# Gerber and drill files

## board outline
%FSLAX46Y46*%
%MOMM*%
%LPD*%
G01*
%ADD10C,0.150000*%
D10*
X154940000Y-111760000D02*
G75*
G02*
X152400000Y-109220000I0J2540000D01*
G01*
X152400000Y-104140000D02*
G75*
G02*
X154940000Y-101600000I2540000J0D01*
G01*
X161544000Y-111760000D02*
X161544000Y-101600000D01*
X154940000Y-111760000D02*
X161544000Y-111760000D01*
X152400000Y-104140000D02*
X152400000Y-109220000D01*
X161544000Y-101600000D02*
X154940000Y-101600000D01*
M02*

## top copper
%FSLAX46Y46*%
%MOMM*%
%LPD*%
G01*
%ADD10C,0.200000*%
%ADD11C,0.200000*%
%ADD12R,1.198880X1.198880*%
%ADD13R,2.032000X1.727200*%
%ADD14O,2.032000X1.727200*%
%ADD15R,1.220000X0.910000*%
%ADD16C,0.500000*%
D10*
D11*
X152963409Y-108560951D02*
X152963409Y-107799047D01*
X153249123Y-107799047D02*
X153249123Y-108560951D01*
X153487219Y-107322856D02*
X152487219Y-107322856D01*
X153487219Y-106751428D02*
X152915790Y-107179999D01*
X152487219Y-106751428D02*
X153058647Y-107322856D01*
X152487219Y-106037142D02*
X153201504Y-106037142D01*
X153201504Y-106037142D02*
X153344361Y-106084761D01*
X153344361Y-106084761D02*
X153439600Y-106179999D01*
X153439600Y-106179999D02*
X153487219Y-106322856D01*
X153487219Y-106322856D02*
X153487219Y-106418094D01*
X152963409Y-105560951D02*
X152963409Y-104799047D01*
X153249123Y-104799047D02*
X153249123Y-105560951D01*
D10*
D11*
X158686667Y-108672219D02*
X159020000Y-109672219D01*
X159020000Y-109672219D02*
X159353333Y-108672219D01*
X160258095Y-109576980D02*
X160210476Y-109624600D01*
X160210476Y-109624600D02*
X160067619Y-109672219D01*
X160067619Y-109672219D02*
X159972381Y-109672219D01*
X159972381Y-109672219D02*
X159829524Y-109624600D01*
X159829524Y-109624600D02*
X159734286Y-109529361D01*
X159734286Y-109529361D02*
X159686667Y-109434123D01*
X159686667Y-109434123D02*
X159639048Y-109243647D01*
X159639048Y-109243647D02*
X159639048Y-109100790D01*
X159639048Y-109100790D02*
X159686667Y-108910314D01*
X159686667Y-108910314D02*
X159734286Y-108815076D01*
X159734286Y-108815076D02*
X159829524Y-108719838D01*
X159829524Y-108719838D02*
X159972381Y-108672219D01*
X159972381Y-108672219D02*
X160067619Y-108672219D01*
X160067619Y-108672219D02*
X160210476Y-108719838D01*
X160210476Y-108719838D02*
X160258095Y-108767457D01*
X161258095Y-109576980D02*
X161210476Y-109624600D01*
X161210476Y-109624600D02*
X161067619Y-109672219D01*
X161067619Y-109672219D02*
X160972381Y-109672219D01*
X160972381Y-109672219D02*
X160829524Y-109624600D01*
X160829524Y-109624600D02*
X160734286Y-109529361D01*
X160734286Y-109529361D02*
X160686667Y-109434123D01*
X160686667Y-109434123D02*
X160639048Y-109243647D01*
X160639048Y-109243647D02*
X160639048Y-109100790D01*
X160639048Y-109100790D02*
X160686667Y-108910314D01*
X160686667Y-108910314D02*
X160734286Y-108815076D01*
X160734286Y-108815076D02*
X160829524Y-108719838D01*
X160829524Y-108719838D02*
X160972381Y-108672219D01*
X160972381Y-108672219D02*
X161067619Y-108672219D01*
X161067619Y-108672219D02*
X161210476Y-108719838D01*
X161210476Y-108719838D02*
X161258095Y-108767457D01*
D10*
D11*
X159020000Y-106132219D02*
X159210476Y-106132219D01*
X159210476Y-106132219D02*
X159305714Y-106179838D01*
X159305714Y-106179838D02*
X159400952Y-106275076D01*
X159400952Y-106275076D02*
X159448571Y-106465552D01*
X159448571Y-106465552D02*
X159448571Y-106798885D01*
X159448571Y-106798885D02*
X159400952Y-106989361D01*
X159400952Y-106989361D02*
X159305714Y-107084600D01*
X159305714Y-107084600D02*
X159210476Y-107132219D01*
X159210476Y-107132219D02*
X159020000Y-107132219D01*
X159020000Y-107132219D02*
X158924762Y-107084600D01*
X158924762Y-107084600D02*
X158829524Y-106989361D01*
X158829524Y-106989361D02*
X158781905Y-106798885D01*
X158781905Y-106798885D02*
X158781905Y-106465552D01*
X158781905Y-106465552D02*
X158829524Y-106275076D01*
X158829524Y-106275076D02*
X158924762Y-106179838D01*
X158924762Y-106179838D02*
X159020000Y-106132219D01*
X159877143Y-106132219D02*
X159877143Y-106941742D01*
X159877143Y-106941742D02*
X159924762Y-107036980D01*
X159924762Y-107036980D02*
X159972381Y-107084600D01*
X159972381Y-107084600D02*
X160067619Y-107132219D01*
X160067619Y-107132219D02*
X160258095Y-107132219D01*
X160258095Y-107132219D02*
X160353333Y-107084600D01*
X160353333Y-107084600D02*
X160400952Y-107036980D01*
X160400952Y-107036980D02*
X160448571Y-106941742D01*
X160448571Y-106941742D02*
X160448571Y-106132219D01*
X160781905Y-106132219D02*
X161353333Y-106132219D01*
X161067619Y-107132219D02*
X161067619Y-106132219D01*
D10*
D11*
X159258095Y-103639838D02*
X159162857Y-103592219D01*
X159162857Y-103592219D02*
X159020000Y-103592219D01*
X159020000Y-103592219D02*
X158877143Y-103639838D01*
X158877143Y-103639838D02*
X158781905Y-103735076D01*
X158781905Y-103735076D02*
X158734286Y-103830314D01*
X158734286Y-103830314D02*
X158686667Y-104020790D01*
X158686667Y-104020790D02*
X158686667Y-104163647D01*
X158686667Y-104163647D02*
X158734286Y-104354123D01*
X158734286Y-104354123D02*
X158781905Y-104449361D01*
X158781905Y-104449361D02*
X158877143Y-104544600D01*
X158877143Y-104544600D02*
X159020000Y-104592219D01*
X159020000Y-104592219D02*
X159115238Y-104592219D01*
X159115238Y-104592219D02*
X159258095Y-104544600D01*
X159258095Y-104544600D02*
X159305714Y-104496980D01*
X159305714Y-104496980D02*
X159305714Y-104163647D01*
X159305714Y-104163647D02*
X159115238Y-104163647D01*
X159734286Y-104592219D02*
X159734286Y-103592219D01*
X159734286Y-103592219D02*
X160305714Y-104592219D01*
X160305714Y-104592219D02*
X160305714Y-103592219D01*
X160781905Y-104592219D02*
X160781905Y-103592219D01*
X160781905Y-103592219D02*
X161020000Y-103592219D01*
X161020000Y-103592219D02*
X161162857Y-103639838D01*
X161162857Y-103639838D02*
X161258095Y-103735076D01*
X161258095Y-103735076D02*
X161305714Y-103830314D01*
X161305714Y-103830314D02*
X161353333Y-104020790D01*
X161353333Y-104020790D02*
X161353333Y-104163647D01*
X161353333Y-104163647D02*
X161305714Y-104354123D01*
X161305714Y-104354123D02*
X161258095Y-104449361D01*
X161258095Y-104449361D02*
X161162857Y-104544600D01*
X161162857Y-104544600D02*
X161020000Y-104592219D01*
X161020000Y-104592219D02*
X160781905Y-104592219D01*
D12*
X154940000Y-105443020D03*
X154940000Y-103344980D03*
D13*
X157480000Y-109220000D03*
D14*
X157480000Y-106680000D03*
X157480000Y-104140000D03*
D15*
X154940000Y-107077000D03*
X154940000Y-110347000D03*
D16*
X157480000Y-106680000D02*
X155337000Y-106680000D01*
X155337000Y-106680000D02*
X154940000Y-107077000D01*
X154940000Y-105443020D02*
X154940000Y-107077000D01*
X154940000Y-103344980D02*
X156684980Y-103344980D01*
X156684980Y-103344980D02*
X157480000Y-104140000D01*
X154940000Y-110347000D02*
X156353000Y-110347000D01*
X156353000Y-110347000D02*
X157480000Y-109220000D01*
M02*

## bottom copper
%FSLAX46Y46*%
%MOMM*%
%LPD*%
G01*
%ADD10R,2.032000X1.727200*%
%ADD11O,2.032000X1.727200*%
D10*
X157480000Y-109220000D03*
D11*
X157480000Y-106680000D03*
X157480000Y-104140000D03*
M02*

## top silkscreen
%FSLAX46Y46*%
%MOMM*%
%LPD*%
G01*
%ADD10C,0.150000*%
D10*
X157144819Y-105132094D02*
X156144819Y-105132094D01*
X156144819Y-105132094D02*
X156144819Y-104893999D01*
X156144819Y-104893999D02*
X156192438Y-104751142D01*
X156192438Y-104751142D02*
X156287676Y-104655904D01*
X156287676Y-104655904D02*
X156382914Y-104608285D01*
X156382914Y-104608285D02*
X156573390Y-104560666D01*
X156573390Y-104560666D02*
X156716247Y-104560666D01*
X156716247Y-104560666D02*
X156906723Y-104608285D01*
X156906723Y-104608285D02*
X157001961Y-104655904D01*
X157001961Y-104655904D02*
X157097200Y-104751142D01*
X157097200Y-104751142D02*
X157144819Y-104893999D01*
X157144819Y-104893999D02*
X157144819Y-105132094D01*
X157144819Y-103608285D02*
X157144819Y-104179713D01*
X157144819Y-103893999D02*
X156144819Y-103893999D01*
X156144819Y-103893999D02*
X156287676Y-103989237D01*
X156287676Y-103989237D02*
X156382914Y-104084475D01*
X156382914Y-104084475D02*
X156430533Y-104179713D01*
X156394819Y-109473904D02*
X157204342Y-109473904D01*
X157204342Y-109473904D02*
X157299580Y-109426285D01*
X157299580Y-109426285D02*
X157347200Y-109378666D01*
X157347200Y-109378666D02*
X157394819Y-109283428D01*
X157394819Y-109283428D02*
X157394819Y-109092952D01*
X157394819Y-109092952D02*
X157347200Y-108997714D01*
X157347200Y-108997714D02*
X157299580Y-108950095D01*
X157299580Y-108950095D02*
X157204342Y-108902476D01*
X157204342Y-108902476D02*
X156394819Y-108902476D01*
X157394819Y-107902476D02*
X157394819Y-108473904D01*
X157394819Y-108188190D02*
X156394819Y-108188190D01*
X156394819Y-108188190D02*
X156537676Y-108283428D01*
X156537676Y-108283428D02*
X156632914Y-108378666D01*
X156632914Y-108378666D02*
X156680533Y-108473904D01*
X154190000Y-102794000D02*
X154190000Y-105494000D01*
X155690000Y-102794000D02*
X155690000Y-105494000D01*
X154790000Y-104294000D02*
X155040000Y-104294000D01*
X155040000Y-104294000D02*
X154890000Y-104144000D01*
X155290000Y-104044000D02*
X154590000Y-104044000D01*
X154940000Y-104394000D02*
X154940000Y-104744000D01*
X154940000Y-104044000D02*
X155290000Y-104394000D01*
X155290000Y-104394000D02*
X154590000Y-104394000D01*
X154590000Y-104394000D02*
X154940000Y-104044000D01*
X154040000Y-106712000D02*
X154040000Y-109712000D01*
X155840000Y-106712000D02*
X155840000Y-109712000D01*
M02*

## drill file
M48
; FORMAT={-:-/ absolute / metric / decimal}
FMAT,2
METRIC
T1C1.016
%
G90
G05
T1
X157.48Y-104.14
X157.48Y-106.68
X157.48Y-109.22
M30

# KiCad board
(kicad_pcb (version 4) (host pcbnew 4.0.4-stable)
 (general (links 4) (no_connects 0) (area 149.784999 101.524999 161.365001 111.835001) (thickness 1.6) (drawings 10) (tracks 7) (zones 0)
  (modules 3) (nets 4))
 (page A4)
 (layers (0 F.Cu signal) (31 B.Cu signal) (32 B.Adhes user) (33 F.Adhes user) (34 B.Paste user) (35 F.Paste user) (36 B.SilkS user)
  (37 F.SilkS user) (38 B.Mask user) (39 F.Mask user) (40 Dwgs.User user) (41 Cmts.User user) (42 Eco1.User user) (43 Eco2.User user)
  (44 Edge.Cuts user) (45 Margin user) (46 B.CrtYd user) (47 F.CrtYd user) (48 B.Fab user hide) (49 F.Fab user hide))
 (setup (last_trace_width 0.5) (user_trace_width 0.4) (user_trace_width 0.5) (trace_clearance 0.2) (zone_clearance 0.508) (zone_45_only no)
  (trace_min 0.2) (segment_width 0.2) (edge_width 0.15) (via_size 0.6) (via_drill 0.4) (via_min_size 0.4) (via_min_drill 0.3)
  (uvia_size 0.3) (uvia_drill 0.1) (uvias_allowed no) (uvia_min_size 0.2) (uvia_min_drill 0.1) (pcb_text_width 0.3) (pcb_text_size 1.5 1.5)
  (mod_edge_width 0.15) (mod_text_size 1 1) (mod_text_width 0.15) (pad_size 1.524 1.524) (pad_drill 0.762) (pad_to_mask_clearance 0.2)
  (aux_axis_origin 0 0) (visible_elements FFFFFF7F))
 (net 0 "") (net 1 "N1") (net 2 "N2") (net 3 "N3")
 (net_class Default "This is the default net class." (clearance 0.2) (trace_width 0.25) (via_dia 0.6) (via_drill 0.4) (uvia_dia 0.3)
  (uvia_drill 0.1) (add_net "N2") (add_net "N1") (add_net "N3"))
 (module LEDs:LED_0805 (layer F.Cu) (at 154.94 104.394 270)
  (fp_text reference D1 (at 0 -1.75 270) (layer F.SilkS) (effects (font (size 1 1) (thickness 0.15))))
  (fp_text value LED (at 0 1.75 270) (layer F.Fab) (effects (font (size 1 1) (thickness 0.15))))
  (fp_line (start -1.6 0.75) (end 1.1 0.75) (layer F.SilkS) (width 0.15))
  (fp_line (start -1.6 -0.75) (end 1.1 -0.75) (layer F.SilkS) (width 0.15))
  (fp_line (start -0.1 0.15) (end -0.1 -0.1) (layer F.SilkS) (width 0.15))
  (fp_line (start -0.1 -0.1) (end -0.25 0.05) (layer F.SilkS) (width 0.15))
  (fp_line (start -0.35 -0.35) (end -0.35 0.35) (layer F.SilkS) (width 0.15))
  (fp_line (start 0 0) (end 0.35 0) (layer F.SilkS) (width 0.15))
  (fp_line (start -0.35 0) (end 0 -0.35) (layer F.SilkS) (width 0.15))
  (fp_line (start 0 -0.35) (end 0 0.35) (layer F.SilkS) (width 0.15))
  (fp_line (start 0 0.35) (end -0.35 0) (layer F.SilkS) (width 0.15))
  (pad 2 smd rect (at 1.04902 0 90) (size 1.19888 1.19888) (layers F.Cu F.Paste F.Mask) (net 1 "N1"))
  (pad 1 smd rect (at -1.04902 0 90) (size 1.19888 1.19888) (layers F.Cu F.Paste F.Mask) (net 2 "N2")))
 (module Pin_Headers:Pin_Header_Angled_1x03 (layer B.Cu) (at 157.48 109.22)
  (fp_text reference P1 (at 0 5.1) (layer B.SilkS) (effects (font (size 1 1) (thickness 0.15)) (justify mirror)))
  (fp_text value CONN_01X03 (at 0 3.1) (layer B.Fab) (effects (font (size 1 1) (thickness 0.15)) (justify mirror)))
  (pad 1 thru_hole rect (at 0 0) (size 2.032 1.7272) (drill 1.016) (layers *.Cu *.Mask) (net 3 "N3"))
  (pad 2 thru_hole oval (at 0 -2.54) (size 2.032 1.7272) (drill 1.016) (layers *.Cu *.Mask) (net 1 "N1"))
  (pad 3 thru_hole oval (at 0 -5.08) (size 2.032 1.7272) (drill 1.016) (layers *.Cu *.Mask) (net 2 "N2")))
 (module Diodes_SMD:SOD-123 (layer F.Cu) (at 154.94 108.712 270)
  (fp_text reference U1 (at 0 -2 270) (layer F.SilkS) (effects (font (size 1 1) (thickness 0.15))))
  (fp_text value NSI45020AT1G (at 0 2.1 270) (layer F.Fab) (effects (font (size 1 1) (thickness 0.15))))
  (fp_line (start -2 0.9) (end 1 0.9) (layer F.SilkS) (width 0.15))
  (fp_line (start -2 -0.9) (end 1 -0.9) (layer F.SilkS) (width 0.15))
  (pad 1 smd rect (at -1.635 0 270) (size 0.91 1.22) (layers F.Cu F.Paste F.Mask) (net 1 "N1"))
  (pad 2 smd rect (at 1.635 0 270) (size 0.91 1.22) (layers F.Cu F.Paste F.Mask) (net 3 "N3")))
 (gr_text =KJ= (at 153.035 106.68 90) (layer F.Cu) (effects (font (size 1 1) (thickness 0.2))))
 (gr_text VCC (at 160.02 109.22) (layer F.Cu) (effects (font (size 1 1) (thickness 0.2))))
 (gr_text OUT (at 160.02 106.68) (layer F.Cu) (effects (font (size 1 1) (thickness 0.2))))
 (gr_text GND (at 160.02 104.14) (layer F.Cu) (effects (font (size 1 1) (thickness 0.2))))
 (gr_arc (start 154.94 109.22) (end 154.94 111.76) (angle 90) (layer Edge.Cuts) (width 0.15))
 (gr_arc (start 154.94 104.14) (end 152.4 104.14) (angle 90) (layer Edge.Cuts) (width 0.15))
 (gr_line (start 161.544 111.76) (end 161.544 101.6) (layer Edge.Cuts) (width 0.15))
 (gr_line (start 154.94 111.76) (end 161.544 111.76) (layer Edge.Cuts) (width 0.15))
 (gr_line (start 152.4 104.14) (end 152.4 109.22) (layer Edge.Cuts) (width 0.15))
 (gr_line (start 161.544 101.6) (end 154.94 101.6) (layer Edge.Cuts) (width 0.15))
 (segment (start 157.48 106.68) (end 155.337 106.68) (width 0.5) (layer F.Cu) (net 1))
 (segment (start 155.337 106.68) (end 154.94 107.077) (width 0.5) (layer F.Cu) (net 1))
 (segment (start 154.94 105.44302) (end 154.94 107.077) (width 0.5) (layer F.Cu) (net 1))
 (segment (start 154.94 103.34498) (end 156.68498 103.34498) (width 0.5) (layer F.Cu) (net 2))
 (segment (start 156.68498 103.34498) (end 157.48 104.14) (width 0.5) (layer F.Cu) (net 2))
 (segment (start 154.94 110.347) (end 156.353 110.347) (width 0.5) (layer F.Cu) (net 3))
 (segment (start 156.353 110.347) (end 157.48 109.22) (width 0.5) (layer F.Cu) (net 3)))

